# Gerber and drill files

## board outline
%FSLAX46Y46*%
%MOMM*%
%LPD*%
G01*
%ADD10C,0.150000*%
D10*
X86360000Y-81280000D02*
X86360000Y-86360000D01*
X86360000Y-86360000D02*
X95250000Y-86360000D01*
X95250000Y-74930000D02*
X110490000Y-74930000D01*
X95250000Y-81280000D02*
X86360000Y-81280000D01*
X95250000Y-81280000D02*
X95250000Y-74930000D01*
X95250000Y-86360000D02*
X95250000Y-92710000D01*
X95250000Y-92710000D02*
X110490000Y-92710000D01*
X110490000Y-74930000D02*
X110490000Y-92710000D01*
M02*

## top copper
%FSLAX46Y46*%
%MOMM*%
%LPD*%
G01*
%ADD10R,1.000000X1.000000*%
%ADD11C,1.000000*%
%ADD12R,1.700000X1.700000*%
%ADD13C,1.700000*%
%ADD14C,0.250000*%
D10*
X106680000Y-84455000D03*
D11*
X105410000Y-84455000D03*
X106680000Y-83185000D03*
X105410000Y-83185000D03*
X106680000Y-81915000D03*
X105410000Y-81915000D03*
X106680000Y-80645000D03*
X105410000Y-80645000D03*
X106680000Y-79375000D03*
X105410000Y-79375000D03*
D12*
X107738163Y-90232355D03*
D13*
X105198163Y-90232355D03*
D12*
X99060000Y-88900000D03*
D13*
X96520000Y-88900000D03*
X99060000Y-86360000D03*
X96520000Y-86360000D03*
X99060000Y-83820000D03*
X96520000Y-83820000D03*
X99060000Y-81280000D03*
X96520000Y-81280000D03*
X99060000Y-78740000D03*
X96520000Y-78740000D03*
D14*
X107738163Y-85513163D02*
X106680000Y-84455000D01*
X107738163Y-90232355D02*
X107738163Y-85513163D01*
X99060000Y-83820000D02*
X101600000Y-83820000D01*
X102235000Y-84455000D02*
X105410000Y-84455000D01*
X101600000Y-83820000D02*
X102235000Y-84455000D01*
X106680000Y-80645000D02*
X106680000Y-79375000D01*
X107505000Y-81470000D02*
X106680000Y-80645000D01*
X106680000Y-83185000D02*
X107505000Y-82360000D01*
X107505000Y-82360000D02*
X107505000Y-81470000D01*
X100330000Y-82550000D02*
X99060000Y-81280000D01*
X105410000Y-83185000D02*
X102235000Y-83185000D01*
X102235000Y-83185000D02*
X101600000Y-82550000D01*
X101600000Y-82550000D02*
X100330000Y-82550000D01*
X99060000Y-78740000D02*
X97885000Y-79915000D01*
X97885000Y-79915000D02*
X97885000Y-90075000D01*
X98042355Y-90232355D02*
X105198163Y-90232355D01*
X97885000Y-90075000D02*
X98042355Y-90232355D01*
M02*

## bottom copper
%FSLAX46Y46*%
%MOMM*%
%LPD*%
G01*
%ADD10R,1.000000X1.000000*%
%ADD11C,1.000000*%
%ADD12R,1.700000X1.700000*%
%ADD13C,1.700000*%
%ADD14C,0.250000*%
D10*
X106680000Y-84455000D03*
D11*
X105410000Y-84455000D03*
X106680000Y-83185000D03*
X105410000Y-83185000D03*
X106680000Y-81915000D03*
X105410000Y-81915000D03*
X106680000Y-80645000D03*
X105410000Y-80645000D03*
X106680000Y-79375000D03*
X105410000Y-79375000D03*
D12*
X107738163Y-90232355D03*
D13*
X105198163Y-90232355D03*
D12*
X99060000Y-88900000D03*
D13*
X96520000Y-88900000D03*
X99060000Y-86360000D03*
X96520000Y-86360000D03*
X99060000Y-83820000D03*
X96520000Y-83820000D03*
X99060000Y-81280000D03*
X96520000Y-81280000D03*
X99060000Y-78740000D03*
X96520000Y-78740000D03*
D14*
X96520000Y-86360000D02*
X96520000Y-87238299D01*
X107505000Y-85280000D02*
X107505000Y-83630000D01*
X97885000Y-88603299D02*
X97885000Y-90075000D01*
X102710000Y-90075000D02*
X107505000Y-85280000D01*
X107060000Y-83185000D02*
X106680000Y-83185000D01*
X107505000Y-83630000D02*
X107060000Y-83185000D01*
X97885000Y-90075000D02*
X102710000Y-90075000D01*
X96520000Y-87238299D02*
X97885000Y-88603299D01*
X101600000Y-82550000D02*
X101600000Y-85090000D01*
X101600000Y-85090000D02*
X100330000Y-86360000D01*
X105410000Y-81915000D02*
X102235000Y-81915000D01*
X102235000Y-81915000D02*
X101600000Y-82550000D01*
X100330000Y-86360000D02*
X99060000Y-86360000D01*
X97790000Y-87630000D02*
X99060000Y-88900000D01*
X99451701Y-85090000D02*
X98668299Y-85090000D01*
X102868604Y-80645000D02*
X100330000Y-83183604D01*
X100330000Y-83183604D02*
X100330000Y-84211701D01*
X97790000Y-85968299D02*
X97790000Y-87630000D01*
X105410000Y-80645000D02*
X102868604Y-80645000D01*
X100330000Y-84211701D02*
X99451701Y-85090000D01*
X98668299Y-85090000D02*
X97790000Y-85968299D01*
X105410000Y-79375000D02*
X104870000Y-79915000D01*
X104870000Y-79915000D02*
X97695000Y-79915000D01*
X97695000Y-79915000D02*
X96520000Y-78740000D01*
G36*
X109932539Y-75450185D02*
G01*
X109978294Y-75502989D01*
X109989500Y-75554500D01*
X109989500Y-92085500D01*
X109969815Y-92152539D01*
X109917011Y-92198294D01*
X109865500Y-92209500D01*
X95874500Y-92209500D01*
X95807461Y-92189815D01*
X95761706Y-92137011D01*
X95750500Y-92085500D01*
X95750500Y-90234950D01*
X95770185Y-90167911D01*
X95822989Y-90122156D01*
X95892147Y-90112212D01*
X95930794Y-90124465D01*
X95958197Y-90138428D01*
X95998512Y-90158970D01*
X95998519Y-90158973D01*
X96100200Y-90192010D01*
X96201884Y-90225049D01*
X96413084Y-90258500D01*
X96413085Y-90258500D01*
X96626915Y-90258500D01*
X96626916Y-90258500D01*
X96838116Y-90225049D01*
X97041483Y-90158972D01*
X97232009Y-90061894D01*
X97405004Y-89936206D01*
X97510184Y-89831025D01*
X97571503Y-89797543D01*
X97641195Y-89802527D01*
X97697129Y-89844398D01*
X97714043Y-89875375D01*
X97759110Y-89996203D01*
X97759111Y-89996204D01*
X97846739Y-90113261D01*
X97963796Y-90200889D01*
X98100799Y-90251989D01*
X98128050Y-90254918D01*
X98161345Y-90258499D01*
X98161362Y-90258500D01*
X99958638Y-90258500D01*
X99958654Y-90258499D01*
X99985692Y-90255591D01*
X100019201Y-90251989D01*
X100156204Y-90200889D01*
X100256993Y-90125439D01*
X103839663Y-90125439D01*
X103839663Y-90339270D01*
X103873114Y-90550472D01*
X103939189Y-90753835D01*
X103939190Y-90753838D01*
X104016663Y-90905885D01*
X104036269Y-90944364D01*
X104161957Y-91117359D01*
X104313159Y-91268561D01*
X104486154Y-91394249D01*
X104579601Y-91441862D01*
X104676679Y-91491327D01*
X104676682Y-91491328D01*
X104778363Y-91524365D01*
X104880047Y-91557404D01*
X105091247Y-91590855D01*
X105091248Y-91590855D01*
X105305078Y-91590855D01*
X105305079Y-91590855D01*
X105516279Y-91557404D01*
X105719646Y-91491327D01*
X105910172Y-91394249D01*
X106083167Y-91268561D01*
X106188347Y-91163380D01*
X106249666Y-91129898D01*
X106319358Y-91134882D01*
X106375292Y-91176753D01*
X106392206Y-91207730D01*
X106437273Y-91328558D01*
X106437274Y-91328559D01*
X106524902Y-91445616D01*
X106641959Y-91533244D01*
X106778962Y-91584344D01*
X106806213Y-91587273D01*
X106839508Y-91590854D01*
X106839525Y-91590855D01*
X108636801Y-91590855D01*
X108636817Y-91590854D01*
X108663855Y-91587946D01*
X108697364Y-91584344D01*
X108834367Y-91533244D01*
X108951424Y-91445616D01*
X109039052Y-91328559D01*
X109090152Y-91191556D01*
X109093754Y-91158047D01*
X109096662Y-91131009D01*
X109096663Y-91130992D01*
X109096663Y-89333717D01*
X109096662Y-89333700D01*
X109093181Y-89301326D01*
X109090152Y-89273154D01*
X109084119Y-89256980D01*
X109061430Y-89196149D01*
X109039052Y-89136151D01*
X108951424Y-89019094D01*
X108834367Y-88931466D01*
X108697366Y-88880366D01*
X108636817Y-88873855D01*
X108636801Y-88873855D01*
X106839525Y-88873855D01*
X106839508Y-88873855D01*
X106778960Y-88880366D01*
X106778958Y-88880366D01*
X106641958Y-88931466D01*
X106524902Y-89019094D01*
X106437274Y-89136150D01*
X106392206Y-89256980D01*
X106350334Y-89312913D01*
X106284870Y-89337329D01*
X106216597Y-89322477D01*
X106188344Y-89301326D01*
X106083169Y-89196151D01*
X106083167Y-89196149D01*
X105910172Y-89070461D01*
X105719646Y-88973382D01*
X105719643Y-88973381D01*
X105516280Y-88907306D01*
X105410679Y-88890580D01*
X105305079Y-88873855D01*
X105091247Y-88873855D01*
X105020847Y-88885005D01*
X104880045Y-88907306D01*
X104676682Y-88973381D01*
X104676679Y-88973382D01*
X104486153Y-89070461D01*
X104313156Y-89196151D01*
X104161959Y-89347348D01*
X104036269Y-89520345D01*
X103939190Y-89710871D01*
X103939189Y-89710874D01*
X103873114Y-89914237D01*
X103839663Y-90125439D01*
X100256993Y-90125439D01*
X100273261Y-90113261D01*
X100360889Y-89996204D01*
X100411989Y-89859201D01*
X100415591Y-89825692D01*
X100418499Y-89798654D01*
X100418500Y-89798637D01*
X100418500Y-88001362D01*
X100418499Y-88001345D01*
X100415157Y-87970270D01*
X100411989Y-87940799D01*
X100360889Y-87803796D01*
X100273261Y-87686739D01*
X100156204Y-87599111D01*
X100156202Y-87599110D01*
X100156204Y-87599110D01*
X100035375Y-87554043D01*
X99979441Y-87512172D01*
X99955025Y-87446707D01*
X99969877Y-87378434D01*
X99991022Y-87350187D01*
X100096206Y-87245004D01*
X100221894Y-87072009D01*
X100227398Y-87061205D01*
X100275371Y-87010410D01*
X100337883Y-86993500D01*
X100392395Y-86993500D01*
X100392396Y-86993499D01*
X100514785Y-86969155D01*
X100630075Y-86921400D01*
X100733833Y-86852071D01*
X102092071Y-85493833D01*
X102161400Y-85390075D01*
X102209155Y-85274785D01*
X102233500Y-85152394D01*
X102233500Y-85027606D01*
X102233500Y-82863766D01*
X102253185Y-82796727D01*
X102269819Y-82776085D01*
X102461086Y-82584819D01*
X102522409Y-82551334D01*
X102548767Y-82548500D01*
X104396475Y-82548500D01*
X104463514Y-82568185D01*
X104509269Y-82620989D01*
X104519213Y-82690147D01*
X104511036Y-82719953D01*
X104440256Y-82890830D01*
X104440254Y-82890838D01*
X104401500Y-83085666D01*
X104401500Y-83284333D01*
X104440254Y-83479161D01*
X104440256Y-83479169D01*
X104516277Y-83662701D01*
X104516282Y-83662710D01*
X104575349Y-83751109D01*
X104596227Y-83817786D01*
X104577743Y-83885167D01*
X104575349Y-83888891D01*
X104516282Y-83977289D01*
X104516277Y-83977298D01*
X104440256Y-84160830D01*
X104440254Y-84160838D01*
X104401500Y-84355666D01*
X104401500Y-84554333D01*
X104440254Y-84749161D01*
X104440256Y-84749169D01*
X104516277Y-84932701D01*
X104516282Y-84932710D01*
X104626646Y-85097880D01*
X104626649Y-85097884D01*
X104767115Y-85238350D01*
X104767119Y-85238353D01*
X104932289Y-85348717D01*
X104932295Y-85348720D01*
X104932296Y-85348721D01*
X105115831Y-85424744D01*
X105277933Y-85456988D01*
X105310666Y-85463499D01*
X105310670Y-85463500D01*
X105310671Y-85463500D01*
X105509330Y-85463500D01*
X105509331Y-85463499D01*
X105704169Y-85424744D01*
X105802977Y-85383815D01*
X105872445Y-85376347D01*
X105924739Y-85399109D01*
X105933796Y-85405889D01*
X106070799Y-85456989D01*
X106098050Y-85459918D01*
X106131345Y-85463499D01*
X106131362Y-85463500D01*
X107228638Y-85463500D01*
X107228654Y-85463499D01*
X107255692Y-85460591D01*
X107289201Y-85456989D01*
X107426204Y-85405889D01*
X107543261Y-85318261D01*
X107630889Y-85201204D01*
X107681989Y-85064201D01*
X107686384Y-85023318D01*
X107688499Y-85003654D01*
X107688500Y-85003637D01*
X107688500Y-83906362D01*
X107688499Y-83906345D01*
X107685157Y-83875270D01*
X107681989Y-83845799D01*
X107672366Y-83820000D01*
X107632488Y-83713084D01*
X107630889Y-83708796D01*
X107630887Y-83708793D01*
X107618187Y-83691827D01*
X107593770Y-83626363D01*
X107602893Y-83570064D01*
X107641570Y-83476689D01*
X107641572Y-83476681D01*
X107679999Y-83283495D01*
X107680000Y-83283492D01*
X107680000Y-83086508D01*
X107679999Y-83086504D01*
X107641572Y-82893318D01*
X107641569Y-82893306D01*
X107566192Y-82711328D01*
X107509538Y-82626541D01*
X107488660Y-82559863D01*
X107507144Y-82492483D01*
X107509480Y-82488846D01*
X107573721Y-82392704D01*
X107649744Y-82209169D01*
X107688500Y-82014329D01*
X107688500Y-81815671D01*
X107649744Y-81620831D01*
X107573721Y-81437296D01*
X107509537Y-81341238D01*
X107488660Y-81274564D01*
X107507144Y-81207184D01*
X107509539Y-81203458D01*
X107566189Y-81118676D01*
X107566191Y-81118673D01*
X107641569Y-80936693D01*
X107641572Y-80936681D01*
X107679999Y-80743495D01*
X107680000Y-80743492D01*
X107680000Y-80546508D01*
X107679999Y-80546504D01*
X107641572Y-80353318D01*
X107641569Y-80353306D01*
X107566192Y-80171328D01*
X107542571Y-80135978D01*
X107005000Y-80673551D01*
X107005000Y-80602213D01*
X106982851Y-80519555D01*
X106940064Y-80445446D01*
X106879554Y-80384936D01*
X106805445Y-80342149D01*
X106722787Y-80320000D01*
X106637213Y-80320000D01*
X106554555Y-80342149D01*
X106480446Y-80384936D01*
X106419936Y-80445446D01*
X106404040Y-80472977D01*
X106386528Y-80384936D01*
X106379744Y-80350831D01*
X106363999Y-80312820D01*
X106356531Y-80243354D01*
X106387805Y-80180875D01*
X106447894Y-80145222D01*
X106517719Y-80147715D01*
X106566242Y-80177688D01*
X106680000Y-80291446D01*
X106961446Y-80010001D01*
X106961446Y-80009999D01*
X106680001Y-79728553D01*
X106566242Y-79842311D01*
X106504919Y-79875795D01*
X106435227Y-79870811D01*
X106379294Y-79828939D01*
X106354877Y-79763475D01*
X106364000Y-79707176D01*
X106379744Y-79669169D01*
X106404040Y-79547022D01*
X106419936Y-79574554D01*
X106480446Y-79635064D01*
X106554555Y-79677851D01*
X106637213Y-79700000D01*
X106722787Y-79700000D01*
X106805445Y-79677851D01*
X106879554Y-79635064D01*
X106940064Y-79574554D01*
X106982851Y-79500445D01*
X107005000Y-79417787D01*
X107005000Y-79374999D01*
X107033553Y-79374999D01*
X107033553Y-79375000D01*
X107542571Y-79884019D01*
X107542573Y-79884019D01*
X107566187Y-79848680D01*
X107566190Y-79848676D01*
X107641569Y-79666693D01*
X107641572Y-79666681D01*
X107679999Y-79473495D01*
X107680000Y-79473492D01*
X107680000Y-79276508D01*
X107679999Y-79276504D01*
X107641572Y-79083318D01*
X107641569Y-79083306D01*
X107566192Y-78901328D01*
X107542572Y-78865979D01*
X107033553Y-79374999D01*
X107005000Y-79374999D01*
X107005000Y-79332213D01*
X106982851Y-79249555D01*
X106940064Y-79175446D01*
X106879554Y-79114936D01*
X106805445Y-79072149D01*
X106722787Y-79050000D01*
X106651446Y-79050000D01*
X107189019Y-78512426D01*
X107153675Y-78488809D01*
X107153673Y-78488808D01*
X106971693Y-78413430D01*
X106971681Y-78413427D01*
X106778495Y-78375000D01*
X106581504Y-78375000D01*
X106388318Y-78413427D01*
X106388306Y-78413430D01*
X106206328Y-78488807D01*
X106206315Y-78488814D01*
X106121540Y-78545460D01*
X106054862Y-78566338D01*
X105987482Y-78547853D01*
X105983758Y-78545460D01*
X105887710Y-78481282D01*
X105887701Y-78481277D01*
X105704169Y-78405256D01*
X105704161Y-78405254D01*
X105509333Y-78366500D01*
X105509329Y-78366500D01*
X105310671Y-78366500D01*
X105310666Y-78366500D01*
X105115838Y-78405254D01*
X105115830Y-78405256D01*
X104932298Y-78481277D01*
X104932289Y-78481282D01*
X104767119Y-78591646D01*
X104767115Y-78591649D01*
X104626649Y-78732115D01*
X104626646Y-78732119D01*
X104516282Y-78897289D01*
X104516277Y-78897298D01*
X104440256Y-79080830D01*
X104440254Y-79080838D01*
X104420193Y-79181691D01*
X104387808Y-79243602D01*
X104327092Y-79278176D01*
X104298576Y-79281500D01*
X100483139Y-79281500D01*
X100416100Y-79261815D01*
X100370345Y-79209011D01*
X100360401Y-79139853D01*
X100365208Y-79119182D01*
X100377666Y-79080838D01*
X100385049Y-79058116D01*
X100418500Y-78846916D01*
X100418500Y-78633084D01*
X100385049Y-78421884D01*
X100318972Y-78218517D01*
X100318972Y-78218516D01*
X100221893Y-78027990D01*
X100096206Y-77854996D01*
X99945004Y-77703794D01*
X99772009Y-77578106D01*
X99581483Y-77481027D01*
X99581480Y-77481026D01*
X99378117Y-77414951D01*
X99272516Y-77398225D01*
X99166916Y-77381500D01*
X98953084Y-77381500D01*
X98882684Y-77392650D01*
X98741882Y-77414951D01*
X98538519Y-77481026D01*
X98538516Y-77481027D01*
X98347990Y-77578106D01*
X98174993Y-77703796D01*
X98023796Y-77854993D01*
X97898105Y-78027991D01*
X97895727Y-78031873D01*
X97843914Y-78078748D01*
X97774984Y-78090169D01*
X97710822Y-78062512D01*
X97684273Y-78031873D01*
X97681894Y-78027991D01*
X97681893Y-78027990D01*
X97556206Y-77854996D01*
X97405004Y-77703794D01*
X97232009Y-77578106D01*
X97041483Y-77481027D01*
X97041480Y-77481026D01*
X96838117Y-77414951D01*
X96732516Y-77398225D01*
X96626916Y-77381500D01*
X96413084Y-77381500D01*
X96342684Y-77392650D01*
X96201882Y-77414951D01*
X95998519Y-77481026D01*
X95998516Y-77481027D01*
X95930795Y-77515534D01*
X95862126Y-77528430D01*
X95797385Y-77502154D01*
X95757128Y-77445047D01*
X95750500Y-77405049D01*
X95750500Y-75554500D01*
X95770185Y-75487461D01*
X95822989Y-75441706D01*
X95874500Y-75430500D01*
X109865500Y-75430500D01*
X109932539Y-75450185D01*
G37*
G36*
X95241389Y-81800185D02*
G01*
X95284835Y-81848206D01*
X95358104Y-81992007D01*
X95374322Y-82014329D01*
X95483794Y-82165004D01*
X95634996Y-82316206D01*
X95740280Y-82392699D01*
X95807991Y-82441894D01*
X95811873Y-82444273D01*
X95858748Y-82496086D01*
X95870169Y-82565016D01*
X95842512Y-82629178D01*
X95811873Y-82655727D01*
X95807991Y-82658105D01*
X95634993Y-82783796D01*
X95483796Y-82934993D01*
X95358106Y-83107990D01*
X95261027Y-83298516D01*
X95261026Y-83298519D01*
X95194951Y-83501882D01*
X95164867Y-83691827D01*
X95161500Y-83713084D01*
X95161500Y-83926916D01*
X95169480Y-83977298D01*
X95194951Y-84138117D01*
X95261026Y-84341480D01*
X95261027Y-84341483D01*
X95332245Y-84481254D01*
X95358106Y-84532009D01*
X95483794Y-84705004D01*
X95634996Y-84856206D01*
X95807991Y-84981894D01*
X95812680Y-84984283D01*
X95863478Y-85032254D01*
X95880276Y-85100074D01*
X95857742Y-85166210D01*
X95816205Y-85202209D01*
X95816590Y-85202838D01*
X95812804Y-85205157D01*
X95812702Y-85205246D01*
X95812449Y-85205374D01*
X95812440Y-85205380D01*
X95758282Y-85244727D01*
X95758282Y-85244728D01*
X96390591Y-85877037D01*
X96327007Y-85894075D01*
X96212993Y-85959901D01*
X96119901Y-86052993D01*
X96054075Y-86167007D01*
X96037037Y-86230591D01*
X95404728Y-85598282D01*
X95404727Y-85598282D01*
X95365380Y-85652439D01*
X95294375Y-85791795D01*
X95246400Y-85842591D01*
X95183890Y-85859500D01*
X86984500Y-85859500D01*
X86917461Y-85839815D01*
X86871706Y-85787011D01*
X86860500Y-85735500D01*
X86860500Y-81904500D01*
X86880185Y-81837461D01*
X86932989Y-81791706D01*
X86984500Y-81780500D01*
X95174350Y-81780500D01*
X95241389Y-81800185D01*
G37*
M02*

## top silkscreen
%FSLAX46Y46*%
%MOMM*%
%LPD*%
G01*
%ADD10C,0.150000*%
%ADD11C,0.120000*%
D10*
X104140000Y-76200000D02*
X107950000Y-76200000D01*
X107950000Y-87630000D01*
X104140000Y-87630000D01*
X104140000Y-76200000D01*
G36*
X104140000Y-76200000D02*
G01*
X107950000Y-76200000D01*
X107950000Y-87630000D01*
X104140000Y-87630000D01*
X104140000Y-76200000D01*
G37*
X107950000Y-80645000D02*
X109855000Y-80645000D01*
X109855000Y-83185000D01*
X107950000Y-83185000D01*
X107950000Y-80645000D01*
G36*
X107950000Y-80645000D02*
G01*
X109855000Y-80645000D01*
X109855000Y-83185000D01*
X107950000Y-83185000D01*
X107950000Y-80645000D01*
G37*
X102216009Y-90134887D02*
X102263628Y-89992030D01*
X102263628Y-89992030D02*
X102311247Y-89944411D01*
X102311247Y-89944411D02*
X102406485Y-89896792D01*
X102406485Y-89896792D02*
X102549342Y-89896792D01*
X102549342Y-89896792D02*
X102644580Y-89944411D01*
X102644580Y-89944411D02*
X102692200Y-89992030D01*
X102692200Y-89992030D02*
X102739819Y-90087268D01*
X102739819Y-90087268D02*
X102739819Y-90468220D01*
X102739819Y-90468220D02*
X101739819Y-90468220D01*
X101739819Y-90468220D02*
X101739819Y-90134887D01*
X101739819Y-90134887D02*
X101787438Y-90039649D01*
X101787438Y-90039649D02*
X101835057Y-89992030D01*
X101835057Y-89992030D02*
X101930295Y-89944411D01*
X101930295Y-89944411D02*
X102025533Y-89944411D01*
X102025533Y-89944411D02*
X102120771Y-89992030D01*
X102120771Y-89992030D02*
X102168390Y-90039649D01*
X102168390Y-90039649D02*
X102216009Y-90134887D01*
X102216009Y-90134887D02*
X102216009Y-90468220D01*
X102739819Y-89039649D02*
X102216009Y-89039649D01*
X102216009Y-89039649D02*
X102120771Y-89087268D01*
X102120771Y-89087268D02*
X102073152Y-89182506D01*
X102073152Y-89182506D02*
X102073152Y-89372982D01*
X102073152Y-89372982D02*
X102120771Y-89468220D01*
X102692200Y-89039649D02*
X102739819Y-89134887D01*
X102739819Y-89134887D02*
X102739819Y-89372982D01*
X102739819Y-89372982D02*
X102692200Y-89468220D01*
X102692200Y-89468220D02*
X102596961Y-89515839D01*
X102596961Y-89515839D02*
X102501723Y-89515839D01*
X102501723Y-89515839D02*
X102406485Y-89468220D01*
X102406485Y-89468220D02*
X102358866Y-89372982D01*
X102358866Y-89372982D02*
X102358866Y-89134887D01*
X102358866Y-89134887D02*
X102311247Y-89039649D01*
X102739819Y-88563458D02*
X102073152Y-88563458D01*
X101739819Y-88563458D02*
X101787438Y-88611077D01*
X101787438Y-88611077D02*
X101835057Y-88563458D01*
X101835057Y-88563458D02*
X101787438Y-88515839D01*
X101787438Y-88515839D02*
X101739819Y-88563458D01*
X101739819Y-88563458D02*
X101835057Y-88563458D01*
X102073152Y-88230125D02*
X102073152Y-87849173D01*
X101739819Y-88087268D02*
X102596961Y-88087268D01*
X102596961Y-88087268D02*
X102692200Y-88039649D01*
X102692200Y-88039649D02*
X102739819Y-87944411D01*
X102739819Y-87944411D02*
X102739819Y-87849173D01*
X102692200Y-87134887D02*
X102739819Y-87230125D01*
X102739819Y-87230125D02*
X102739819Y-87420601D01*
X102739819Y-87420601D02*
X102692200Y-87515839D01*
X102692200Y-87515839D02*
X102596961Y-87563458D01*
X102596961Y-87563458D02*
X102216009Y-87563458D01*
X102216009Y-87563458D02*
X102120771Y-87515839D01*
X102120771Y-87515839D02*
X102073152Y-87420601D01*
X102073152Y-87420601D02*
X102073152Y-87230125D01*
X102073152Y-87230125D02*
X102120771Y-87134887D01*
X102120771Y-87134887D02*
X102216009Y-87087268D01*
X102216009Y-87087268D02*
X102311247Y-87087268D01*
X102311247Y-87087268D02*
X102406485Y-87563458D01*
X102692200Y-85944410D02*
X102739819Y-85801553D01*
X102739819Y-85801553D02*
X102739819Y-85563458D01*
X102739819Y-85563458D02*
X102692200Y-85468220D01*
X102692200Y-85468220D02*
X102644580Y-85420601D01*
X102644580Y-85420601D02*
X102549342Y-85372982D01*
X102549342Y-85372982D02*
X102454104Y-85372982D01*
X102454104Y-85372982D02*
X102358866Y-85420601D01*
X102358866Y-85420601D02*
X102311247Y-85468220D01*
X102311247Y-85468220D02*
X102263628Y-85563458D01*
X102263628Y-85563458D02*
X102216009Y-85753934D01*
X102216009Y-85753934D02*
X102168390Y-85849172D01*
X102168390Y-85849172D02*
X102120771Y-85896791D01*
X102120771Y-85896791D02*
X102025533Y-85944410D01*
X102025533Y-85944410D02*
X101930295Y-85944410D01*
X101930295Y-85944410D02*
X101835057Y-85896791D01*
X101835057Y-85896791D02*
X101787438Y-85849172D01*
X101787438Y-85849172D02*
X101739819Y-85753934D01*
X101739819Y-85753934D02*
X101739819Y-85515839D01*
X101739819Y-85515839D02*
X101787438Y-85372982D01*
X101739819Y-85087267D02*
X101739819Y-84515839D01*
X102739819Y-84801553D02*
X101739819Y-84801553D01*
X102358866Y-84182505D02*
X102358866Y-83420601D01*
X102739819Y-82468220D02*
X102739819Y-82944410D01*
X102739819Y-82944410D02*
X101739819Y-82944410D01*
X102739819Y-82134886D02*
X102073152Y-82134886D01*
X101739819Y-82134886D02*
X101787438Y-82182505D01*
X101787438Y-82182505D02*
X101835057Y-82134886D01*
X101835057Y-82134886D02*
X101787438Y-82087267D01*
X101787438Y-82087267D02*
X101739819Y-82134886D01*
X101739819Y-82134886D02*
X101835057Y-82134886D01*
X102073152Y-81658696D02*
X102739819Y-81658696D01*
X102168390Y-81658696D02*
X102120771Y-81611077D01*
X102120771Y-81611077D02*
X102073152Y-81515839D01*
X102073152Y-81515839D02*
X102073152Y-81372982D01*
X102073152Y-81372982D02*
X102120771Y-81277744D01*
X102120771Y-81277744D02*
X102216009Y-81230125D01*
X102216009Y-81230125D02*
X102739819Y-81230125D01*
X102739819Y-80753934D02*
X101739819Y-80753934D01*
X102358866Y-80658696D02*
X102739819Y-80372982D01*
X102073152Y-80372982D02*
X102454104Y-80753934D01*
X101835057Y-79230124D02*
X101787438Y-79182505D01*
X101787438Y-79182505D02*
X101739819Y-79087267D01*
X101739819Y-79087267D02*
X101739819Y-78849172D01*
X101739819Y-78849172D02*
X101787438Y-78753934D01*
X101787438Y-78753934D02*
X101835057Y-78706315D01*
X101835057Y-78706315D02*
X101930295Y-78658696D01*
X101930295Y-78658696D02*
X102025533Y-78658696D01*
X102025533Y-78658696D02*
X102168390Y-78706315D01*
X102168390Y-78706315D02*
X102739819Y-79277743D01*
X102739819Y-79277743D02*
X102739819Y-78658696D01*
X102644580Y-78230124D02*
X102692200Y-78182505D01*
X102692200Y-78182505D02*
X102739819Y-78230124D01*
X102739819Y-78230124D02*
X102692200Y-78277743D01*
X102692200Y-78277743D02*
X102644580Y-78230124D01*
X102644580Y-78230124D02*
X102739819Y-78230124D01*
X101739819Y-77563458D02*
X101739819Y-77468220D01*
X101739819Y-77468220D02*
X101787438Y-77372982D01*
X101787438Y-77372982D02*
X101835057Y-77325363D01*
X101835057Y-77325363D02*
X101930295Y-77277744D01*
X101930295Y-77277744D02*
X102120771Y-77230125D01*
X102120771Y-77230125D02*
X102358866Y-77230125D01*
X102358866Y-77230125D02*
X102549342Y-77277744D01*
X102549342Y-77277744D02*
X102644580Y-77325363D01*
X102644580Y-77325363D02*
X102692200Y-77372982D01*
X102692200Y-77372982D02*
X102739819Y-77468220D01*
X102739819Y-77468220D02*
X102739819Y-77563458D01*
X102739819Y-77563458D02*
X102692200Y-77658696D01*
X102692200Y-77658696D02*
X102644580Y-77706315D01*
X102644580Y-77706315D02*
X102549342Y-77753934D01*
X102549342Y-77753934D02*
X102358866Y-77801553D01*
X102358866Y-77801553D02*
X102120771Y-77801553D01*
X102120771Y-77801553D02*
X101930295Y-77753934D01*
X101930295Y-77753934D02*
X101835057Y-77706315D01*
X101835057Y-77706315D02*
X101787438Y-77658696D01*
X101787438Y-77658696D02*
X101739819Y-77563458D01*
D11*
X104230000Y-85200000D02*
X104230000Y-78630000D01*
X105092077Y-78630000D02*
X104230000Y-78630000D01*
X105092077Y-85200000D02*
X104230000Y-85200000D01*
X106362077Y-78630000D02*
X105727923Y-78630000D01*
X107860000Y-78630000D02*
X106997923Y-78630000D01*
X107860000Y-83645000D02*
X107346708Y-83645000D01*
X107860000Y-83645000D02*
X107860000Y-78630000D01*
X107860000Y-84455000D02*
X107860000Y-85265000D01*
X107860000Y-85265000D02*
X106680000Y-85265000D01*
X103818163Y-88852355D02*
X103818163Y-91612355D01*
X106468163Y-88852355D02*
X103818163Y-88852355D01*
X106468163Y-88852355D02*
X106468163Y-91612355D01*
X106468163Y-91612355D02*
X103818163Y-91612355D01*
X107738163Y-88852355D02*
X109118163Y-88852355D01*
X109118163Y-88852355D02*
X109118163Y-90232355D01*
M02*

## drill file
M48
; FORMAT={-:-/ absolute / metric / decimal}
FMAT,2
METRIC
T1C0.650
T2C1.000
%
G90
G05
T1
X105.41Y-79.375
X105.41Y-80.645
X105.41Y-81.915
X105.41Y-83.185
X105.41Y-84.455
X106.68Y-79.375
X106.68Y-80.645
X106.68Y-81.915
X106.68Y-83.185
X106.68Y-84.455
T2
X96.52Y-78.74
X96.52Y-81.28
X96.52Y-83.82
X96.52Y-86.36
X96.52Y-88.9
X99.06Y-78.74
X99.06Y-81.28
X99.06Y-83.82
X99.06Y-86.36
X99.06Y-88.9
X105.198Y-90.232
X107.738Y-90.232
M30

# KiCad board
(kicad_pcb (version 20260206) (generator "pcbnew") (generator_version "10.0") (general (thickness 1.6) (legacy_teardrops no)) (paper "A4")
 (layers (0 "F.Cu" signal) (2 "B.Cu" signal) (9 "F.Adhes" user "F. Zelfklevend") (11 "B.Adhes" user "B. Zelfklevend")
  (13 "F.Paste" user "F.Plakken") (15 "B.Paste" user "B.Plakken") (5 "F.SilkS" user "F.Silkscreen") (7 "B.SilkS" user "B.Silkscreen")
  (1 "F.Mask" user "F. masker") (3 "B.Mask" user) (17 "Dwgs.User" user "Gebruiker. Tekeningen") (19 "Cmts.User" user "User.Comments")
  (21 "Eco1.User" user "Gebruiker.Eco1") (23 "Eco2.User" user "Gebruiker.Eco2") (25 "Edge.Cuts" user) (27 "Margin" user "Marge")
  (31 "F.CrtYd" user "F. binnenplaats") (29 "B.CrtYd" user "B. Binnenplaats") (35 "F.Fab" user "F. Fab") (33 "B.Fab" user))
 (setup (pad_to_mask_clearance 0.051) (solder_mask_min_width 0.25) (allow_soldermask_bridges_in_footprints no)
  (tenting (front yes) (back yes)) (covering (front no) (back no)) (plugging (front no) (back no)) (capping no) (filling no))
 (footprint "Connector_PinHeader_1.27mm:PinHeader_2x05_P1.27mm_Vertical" (layer "F.Cu") (at 106.68 84.455 180)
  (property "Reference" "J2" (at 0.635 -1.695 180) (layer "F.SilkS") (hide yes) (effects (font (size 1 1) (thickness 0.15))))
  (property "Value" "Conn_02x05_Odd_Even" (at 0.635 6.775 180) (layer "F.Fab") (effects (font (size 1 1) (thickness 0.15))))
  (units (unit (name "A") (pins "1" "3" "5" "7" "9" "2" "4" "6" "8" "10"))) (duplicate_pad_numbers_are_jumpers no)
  (fp_line (start 2.45 -0.745) (end 2.45 5.825) (stroke (width 0.12) (type solid)) (layer "F.SilkS"))
  (fp_line (start 1.587923 5.825) (end 2.45 5.825) (stroke (width 0.12) (type solid)) (layer "F.SilkS"))
  (fp_line (start 1.587923 -0.745) (end 2.45 -0.745) (stroke (width 0.12) (type solid)) (layer "F.SilkS"))
  (fp_line (start 0.317923 5.825) (end 0.952077 5.825) (stroke (width 0.12) (type solid)) (layer "F.SilkS"))
  (fp_line (start -1.18 5.825) (end -0.317923 5.825) (stroke (width 0.12) (type solid)) (layer "F.SilkS"))
  (fp_line (start -1.18 0.81) (end -0.666708 0.81) (stroke (width 0.12) (type solid)) (layer "F.SilkS"))
  (fp_line (start -1.18 0.81) (end -1.18 5.825) (stroke (width 0.12) (type solid)) (layer "F.SilkS"))
  (fp_line (start -1.18 0) (end -1.18 -0.81) (stroke (width 0.12) (type solid)) (layer "F.SilkS"))
  (fp_line (start -1.18 -0.81) (end 0 -0.81) (stroke (width 0.12) (type solid)) (layer "F.SilkS"))
  (pad "1" thru_hole rect (at 0 0 180) (size 1 1) (drill 0.65) (layers "*.Cu" "*.Mask") (remove_unused_layers no) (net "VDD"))
  (pad "2" thru_hole circle (at 1.27 0 180) (size 1 1) (drill 0.65) (layers "*.Cu" "*.Mask") (remove_unused_layers no) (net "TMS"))
  (pad "3" thru_hole circle (at 0 1.27 180) (size 1 1) (drill 0.65) (layers "*.Cu" "*.Mask") (remove_unused_layers no) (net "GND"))
  (pad "4" thru_hole circle (at 1.27 1.27 180) (size 1 1) (drill 0.65) (layers "*.Cu" "*.Mask") (remove_unused_layers no) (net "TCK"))
  (pad "5" thru_hole circle (at 0 2.54 180) (size 1 1) (drill 0.65) (layers "*.Cu" "*.Mask") (remove_unused_layers no)
   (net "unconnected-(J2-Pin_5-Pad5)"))
  (pad "6" thru_hole circle (at 1.27 2.54 180) (size 1 1) (drill 0.65) (layers "*.Cu" "*.Mask") (remove_unused_layers no) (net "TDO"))
  (pad "7" thru_hole circle (at 0 3.81 180) (size 1 1) (drill 0.65) (layers "*.Cu" "*.Mask") (remove_unused_layers no) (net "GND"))
  (pad "8" thru_hole circle (at 1.27 3.81 180) (size 1 1) (drill 0.65) (layers "*.Cu" "*.Mask") (remove_unused_layers no) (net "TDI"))
  (pad "9" thru_hole circle (at 0 5.08 180) (size 1 1) (drill 0.65) (layers "*.Cu" "*.Mask") (remove_unused_layers no) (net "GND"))
  (pad "10" thru_hole circle (at 1.27 5.08 180) (size 1 1) (drill 0.65) (layers "*.Cu" "*.Mask") (remove_unused_layers no) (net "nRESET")))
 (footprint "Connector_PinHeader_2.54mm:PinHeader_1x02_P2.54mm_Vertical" (layer "F.Cu") (at 107.738163 90.232355 -90)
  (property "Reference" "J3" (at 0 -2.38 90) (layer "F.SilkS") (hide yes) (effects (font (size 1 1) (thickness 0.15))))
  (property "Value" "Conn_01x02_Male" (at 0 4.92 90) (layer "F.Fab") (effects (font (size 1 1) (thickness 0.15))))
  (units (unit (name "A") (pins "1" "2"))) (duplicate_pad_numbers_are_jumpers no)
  (fp_line (start -1.38 3.92) (end 1.38 3.92) (stroke (width 0.12) (type solid)) (layer "F.SilkS"))
  (fp_line (start -1.38 1.27) (end -1.38 3.92) (stroke (width 0.12) (type solid)) (layer "F.SilkS"))
  (fp_line (start -1.38 1.27) (end 1.38 1.27) (stroke (width 0.12) (type solid)) (layer "F.SilkS"))
  (fp_line (start 1.38 1.27) (end 1.38 3.92) (stroke (width 0.12) (type solid)) (layer "F.SilkS"))
  (fp_line (start -1.38 0) (end -1.38 -1.38) (stroke (width 0.12) (type solid)) (layer "F.SilkS"))
  (fp_line (start -1.38 -1.38) (end 0 -1.38) (stroke (width 0.12) (type solid)) (layer "F.SilkS"))
  (pad "1" thru_hole rect (at 0 0 270) (size 1.7 1.7) (drill 1) (layers "*.Cu" "*.Mask") (remove_unused_layers no) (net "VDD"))
  (pad "2" thru_hole circle (at 0 2.54 270) (size 1.7 1.7) (drill 1) (layers "*.Cu" "*.Mask") (remove_unused_layers no) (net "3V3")))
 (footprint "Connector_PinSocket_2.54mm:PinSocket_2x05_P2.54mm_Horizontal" (layer "B.Cu") (at 99.06 88.9)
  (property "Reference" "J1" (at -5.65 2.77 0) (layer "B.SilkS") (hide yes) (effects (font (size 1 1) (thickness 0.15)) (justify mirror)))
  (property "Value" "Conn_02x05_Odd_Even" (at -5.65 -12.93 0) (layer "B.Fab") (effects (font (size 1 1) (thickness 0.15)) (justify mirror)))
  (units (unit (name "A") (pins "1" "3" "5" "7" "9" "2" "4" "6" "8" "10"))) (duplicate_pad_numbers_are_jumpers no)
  (pad "1" thru_hole rect (at 0 0) (size 1.7 1.7) (drill 1) (layers "*.Cu" "*.Mask") (remove_unused_layers no) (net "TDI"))
  (pad "2" thru_hole circle (at -2.54 0) (size 1.7 1.7) (drill 1) (layers "*.Cu" "*.Mask") (remove_unused_layers no) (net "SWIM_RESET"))
  (pad "3" thru_hole circle (at 0 -2.54) (size 1.7 1.7) (drill 1) (layers "*.Cu" "*.Mask") (remove_unused_layers no) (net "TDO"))
  (pad "4" thru_hole circle (at -2.54 -2.54) (size 1.7 1.7) (drill 1) (layers "*.Cu" "*.Mask") (remove_unused_layers no) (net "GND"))
  (pad "5" thru_hole circle (at 0 -5.08) (size 1.7 1.7) (drill 1) (layers "*.Cu" "*.Mask") (remove_unused_layers no) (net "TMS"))
  (pad "6" thru_hole circle (at -2.54 -5.08) (size 1.7 1.7) (drill 1) (layers "*.Cu" "*.Mask") (remove_unused_layers no) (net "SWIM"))
  (pad "7" thru_hole circle (at 0 -7.62) (size 1.7 1.7) (drill 1) (layers "*.Cu" "*.Mask") (remove_unused_layers no) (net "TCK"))
  (pad "8" thru_hole circle (at -2.54 -7.62) (size 1.7 1.7) (drill 1) (layers "*.Cu" "*.Mask") (remove_unused_layers no) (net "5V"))
  (pad "9" thru_hole circle (at 0 -10.16) (size 1.7 1.7) (drill 1) (layers "*.Cu" "*.Mask") (remove_unused_layers no) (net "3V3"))
  (pad "10" thru_hole circle (at -2.54 -10.16) (size 1.7 1.7) (drill 1) (layers "*.Cu" "*.Mask") (remove_unused_layers no) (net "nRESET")))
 (gr_rect (start 104.14 76.2) (end 107.95 87.63) (stroke (width 0.15) (type solid)) (fill yes) (layer "F.SilkS"))
 (gr_rect (start 107.95 80.645) (end 109.855 83.185) (stroke (width 0.15) (type solid)) (fill yes) (layer "F.SilkS"))
 (gr_line (start 86.36 81.28) (end 86.36 86.36) (stroke (width 0.15) (type default)) (layer "Edge.Cuts"))
 (gr_line (start 86.36 86.36) (end 95.25 86.36) (stroke (width 0.15) (type default)) (layer "Edge.Cuts"))
 (gr_line (start 95.25 74.93) (end 110.49 74.93) (stroke (width 0.15) (type default)) (layer "Edge.Cuts"))
 (gr_line (start 95.25 81.28) (end 86.36 81.28) (stroke (width 0.15) (type default)) (layer "Edge.Cuts"))
 (gr_line (start 95.25 81.28) (end 95.25 74.93) (stroke (width 0.15) (type default)) (layer "Edge.Cuts"))
 (gr_line (start 95.25 86.36) (end 95.25 92.71) (stroke (width 0.15) (type default)) (layer "Edge.Cuts"))
 (gr_line (start 95.25 92.71) (end 110.49 92.71) (stroke (width 0.15) (type default)) (layer "Edge.Cuts"))
 (gr_line (start 110.49 74.93) (end 110.49 92.71) (stroke (width 0.15) (type default)) (layer "Edge.Cuts"))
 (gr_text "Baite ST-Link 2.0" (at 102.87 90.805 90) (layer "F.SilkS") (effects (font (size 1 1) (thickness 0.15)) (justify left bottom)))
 (segment (start 107.738163 85.513163) (end 106.68 84.455) (width 0.25) (layer "F.Cu") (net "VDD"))
 (segment (start 107.738163 90.232355) (end 107.738163 85.513163) (width 0.25) (layer "F.Cu") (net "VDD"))
 (segment (start 99.06 83.82) (end 101.6 83.82) (width 0.25) (layer "F.Cu") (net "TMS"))
 (segment (start 102.235 84.455) (end 105.41 84.455) (width 0.25) (layer "F.Cu") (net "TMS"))
 (segment (start 101.6 83.82) (end 102.235 84.455) (width 0.25) (layer "F.Cu") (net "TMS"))
 (segment (start 106.68 80.645) (end 106.68 79.375) (width 0.25) (layer "F.Cu") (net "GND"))
 (segment (start 107.505 81.47) (end 106.68 80.645) (width 0.25) (layer "F.Cu") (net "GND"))
 (segment (start 106.68 83.185) (end 107.505 82.36) (width 0.25) (layer "F.Cu") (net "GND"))
 (segment (start 107.505 82.36) (end 107.505 81.47) (width 0.25) (layer "F.Cu") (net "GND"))
 (segment (start 96.52 86.36) (end 96.52 87.238299) (width 0.25) (layer "B.Cu") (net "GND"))
 (segment (start 107.505 85.28) (end 107.505 83.63) (width 0.25) (layer "B.Cu") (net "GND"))
 (segment (start 97.885 88.603299) (end 97.885 90.075) (width 0.25) (layer "B.Cu") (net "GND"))
 (segment (start 102.71 90.075) (end 107.505 85.28) (width 0.25) (layer "B.Cu") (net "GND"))
 (segment (start 107.06 83.185) (end 106.68 83.185) (width 0.25) (layer "B.Cu") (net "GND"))
 (segment (start 107.505 83.63) (end 107.06 83.185) (width 0.25) (layer "B.Cu") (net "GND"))
 (segment (start 97.885 90.075) (end 102.71 90.075) (width 0.25) (layer "B.Cu") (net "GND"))
 (segment (start 96.52 87.238299) (end 97.885 88.603299) (width 0.25) (layer "B.Cu") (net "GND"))
 (segment (start 100.33 82.55) (end 99.06 81.28) (width 0.25) (layer "F.Cu") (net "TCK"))
 (segment (start 105.41 83.185) (end 102.235 83.185) (width 0.25) (layer "F.Cu") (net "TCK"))
 (segment (start 102.235 83.185) (end 101.6 82.55) (width 0.25) (layer "F.Cu") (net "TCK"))
 (segment (start 101.6 82.55) (end 100.33 82.55) (width 0.25) (layer "F.Cu") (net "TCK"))
 (segment (start 101.6 82.55) (end 101.6 85.09) (width 0.25) (layer "B.Cu") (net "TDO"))
 (segment (start 101.6 85.09) (end 100.33 86.36) (width 0.25) (layer "B.Cu") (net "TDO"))
 (segment (start 105.41 81.915) (end 102.235 81.915) (width 0.25) (layer "B.Cu") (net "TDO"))
 (segment (start 102.235 81.915) (end 101.6 82.55) (width 0.25) (layer "B.Cu") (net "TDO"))
 (segment (start 100.33 86.36) (end 99.06 86.36) (width 0.25) (layer "B.Cu") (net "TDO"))
 (segment (start 97.79 87.63) (end 99.06 88.9) (width 0.25) (layer "B.Cu") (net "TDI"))
 (segment (start 99.451701 85.09) (end 98.668299 85.09) (width 0.25) (layer "B.Cu") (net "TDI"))
 (segment (start 102.868604 80.645) (end 100.33 83.183604) (width 0.25) (layer "B.Cu") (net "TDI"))
 (segment (start 100.33 83.183604) (end 100.33 84.211701) (width 0.25) (layer "B.Cu") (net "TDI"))
 (segment (start 97.79 85.968299) (end 97.79 87.63) (width 0.25) (layer "B.Cu") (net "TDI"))
 (segment (start 105.41 80.645) (end 102.868604 80.645) (width 0.25) (layer "B.Cu") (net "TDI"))
 (segment (start 100.33 84.211701) (end 99.451701 85.09) (width 0.25) (layer "B.Cu") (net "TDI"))
 (segment (start 98.668299 85.09) (end 97.79 85.968299) (width 0.25) (layer "B.Cu") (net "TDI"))
 (segment (start 105.41 79.375) (end 104.87 79.915) (width 0.25) (layer "B.Cu") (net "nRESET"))
 (segment (start 104.87 79.915) (end 97.695 79.915) (width 0.25) (layer "B.Cu") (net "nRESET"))
 (segment (start 97.695 79.915) (end 96.52 78.74) (width 0.25) (layer "B.Cu") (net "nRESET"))
 (segment (start 99.06 78.74) (end 97.885 79.915) (width 0.25) (layer "F.Cu") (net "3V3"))
 (segment (start 97.885 79.915) (end 97.885 90.075) (width 0.25) (layer "F.Cu") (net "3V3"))
 (segment (start 98.042355 90.232355) (end 105.198163 90.232355) (width 0.25) (layer "F.Cu") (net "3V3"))
 (segment (start 97.885 90.075) (end 98.042355 90.232355) (width 0.25) (layer "F.Cu") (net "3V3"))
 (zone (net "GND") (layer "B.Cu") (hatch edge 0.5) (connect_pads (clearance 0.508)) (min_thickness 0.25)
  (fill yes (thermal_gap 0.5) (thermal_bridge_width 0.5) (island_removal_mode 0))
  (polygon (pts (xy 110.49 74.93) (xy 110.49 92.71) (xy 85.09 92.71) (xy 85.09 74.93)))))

